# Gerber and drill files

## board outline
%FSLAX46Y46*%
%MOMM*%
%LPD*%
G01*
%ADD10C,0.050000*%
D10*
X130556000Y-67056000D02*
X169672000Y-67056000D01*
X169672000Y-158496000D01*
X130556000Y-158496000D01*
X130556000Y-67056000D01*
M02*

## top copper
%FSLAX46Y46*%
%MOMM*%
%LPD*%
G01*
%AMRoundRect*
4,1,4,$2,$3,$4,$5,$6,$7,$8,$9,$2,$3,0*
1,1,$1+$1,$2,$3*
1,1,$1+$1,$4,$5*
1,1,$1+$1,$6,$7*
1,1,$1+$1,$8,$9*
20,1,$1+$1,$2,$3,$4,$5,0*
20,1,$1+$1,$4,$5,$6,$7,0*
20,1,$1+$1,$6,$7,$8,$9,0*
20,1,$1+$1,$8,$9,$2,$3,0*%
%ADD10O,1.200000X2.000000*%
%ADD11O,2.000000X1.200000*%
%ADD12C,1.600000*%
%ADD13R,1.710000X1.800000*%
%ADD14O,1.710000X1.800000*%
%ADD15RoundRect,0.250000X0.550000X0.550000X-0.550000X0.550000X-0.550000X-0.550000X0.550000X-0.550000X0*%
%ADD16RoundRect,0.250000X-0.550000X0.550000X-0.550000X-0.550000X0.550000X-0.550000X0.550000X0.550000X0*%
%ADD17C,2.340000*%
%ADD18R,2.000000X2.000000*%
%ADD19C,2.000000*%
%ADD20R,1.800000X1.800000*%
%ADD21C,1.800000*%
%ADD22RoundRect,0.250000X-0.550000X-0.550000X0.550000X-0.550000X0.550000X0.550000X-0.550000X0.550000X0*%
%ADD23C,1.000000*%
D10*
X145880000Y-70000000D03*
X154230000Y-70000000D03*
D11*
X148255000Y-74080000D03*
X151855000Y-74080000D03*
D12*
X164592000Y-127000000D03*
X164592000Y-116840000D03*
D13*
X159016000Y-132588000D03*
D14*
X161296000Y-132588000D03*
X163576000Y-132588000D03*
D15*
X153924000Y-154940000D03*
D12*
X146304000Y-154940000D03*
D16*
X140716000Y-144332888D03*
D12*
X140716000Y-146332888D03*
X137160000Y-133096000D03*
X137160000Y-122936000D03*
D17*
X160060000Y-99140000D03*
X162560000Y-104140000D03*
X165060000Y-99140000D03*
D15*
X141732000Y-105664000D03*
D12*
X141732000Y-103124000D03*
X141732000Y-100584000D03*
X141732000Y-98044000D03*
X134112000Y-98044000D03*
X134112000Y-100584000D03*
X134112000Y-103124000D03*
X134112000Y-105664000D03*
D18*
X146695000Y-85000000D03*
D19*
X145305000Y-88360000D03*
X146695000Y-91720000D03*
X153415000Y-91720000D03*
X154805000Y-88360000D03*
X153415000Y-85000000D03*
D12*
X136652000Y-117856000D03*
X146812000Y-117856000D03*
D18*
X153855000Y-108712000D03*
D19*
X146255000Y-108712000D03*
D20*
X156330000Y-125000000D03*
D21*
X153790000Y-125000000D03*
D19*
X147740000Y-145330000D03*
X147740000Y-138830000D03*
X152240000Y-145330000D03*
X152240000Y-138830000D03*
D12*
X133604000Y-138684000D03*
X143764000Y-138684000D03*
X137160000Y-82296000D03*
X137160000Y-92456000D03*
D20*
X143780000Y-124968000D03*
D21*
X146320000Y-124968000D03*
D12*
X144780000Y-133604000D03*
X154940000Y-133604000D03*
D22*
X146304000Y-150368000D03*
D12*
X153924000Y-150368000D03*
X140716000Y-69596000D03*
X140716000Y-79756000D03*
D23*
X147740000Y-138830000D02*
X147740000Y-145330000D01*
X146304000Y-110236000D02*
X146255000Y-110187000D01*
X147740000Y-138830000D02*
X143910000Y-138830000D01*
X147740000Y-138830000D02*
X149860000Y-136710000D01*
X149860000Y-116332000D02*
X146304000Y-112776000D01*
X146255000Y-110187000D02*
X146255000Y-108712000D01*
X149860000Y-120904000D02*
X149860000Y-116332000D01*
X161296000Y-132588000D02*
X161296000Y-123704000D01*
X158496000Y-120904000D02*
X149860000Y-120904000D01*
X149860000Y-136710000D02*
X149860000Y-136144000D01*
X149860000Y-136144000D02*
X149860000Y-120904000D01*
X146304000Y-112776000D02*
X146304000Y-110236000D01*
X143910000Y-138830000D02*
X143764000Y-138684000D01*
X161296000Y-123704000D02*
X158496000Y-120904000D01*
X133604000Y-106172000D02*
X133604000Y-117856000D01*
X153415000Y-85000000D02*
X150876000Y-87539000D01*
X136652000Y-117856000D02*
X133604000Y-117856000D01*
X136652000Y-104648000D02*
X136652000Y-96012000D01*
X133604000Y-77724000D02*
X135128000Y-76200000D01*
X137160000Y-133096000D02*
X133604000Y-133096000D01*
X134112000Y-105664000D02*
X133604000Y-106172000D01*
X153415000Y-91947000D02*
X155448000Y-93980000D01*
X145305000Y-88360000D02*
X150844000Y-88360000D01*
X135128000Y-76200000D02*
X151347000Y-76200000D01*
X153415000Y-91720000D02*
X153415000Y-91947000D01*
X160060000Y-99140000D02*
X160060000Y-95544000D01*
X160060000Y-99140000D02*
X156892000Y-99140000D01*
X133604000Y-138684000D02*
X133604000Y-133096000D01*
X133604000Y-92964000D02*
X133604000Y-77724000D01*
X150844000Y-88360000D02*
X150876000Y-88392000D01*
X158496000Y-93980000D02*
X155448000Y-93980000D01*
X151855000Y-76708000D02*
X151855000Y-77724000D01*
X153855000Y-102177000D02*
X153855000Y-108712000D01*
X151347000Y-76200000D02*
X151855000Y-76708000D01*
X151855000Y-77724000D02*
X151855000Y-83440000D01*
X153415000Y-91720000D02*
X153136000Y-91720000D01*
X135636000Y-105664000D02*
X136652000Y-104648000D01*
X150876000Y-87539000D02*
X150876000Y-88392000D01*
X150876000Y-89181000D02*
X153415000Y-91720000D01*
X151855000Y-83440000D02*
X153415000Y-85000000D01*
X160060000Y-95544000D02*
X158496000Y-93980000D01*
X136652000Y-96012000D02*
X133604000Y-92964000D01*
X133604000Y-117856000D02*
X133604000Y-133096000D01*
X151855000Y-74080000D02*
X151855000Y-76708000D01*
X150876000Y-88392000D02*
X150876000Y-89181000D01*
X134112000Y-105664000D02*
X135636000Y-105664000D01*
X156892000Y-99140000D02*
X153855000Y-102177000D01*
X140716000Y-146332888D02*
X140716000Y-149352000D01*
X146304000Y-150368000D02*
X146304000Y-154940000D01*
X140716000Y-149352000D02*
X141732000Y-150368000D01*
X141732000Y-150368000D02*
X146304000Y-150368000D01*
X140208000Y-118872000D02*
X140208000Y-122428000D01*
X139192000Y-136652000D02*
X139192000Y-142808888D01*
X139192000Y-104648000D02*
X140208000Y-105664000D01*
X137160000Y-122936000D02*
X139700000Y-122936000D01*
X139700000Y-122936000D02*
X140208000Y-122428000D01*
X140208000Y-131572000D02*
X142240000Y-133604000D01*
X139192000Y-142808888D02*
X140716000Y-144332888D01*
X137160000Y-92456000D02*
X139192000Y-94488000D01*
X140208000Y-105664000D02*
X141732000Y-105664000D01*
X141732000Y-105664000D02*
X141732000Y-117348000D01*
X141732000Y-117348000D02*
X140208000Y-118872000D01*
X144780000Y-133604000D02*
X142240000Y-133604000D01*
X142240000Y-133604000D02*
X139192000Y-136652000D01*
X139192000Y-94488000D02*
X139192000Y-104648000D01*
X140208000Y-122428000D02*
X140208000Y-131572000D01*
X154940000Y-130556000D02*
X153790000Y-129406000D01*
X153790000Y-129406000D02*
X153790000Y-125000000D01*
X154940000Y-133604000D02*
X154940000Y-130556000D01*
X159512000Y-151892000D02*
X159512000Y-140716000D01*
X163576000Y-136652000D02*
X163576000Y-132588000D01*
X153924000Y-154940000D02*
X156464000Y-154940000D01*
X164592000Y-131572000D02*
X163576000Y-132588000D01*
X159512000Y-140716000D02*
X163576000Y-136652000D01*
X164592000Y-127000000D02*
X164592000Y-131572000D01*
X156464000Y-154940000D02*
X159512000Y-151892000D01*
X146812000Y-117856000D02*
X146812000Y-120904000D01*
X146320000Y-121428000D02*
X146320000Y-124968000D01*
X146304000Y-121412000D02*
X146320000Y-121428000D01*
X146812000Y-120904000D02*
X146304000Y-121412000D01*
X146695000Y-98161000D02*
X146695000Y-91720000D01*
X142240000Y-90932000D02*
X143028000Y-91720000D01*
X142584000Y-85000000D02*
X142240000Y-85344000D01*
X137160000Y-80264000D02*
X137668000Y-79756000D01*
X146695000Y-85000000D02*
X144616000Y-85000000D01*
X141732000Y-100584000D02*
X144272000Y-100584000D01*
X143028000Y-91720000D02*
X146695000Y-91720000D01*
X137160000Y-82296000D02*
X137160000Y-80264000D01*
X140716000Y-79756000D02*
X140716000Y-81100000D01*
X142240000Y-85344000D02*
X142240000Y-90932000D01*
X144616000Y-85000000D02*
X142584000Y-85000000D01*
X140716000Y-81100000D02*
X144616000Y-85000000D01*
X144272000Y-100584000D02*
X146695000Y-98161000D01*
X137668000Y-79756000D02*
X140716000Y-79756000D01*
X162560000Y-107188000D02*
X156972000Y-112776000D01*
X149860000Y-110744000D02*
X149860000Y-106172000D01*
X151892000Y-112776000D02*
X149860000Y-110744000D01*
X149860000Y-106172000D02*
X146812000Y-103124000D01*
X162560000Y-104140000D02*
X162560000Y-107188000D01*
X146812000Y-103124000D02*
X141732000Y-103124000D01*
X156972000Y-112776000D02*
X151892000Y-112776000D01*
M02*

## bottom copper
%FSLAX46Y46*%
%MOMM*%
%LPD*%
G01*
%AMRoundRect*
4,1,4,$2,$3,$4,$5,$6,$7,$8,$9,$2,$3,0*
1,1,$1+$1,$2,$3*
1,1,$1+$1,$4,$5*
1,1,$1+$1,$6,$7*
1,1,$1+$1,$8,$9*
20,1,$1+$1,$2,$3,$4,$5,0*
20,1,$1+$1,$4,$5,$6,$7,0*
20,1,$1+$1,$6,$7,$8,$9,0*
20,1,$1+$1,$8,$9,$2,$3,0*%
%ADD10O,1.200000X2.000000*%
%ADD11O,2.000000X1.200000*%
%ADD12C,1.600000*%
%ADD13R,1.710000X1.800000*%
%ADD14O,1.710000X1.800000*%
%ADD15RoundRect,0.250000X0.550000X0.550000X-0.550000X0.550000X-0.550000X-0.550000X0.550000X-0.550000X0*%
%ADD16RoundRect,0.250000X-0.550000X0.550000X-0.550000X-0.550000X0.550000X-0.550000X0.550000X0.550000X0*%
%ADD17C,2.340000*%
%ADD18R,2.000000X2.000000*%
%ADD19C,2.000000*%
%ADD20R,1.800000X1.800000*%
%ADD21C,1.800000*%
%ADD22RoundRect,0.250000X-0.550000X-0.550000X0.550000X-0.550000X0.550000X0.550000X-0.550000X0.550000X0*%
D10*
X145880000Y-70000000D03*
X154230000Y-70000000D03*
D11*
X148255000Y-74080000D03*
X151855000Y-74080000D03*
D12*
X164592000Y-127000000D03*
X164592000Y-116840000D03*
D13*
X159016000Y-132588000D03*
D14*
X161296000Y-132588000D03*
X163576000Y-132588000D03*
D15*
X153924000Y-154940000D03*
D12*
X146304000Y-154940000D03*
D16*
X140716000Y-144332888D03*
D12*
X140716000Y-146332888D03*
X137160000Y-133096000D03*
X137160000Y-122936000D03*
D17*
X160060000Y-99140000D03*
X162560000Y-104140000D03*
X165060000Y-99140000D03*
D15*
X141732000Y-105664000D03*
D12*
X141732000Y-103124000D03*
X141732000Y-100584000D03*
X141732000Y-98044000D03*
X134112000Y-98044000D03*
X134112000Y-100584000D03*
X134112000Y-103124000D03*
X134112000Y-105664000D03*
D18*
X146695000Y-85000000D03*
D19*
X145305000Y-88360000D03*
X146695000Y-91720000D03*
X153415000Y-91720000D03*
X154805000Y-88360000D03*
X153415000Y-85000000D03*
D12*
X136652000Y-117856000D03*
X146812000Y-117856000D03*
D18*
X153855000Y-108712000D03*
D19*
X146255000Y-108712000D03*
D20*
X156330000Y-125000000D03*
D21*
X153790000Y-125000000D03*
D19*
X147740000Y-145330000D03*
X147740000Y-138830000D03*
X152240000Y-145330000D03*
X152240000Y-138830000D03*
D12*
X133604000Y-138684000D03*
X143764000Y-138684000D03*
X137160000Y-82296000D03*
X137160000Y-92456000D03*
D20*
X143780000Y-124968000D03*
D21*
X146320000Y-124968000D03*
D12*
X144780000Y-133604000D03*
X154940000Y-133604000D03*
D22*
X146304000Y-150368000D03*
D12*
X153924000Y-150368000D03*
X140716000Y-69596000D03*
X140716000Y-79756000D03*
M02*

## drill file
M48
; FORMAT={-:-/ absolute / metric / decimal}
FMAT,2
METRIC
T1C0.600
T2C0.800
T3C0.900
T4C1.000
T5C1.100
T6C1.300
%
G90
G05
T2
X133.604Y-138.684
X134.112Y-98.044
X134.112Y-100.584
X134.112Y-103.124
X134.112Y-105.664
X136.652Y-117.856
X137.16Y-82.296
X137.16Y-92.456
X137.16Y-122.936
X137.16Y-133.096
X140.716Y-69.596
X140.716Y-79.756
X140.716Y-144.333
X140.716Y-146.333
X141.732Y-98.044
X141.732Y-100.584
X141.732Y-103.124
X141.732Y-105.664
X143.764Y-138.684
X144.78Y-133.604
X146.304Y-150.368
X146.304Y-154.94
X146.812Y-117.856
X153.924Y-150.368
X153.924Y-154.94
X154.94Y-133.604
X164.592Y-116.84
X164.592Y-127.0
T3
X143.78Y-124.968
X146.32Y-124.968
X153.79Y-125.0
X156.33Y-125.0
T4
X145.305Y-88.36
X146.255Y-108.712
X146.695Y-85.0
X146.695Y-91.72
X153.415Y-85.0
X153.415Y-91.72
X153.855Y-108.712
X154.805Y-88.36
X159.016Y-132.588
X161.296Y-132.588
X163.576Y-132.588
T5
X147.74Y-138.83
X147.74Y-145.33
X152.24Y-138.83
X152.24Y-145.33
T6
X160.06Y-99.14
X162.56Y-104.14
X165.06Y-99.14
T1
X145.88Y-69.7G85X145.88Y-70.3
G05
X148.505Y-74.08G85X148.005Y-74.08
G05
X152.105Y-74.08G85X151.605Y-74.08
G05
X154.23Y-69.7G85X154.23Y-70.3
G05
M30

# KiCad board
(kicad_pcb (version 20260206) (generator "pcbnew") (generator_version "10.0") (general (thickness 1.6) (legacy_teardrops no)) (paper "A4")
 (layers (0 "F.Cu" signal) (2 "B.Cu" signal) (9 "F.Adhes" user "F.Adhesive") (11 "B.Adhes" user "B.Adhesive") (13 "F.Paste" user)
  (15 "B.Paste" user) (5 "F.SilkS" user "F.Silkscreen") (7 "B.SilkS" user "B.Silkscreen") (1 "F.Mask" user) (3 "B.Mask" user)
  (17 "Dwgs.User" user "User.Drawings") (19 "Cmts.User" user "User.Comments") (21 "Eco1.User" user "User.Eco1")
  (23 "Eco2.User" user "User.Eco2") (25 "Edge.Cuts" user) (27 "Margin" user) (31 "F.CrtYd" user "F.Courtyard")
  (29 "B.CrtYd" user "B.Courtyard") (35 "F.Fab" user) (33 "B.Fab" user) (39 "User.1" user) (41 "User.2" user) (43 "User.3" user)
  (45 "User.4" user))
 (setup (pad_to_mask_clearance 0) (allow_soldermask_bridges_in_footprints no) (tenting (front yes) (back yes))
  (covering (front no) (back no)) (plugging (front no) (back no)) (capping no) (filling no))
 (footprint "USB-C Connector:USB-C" (layer "F.Cu") (at 150.055 70)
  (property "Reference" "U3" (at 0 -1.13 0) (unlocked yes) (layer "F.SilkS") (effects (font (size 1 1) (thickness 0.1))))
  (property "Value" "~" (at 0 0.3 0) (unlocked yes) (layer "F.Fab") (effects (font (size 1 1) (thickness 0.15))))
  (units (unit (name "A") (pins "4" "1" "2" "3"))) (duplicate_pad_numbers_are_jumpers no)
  (pad "1" thru_hole oval (at -4.175 0 270) (size 2 1.2) (drill oval 1.2 0.6) (layers "*.Cu" "*.Mask") (remove_unused_layers no)
   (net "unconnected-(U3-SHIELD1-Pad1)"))
  (pad "2" thru_hole oval (at 4.175 0 270) (size 2 1.2) (drill oval 1.2 0.6) (layers "*.Cu" "*.Mask") (remove_unused_layers no)
   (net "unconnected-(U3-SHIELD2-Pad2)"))
  (pad "3" thru_hole oval (at -1.8 4.08 270) (size 1.2 2) (drill oval 0.6 1.1) (layers "*.Cu" "*.Mask") (remove_unused_layers no)
   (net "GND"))
  (pad "4" thru_hole oval (at 1.8 4.08 270) (size 1.2 2) (drill oval 0.6 1.1) (layers "*.Cu" "*.Mask") (remove_unused_layers no) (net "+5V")))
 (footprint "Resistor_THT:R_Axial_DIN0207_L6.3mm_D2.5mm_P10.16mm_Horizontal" (layer "F.Cu") (at 164.592 127 90)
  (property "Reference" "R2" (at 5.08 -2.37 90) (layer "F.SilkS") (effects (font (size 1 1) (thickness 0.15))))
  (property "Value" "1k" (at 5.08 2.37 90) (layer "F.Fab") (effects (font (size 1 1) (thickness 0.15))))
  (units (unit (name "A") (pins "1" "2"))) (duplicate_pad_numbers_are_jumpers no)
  (pad "1" thru_hole circle (at 0 0 90) (size 1.6 1.6) (drill 0.8) (layers "*.Cu" "*.Mask") (remove_unused_layers no) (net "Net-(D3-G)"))
  (pad "2" thru_hole circle (at 10.16 0 90) (size 1.6 1.6) (drill 0.8) (layers "*.Cu" "*.Mask") (remove_unused_layers no) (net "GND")))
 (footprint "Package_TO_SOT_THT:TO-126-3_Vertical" (layer "F.Cu") (at 159.016 132.588)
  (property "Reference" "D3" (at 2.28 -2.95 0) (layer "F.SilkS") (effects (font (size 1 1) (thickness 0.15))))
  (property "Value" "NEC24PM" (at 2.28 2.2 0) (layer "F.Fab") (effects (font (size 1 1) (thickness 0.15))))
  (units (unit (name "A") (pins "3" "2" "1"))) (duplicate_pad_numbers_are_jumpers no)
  (pad "1" thru_hole rect (at 0 0) (size 1.71 1.8) (drill 1) (layers "*.Cu" "*.Mask") (remove_unused_layers no) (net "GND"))
  (pad "2" thru_hole oval (at 2.28 0) (size 1.71 1.8) (drill 1) (layers "*.Cu" "*.Mask") (remove_unused_layers no) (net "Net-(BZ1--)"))
  (pad "3" thru_hole oval (at 4.56 0) (size 1.71 1.8) (drill 1) (layers "*.Cu" "*.Mask") (remove_unused_layers no) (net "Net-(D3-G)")))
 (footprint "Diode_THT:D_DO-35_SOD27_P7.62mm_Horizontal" (layer "F.Cu") (at 153.924 154.94 180)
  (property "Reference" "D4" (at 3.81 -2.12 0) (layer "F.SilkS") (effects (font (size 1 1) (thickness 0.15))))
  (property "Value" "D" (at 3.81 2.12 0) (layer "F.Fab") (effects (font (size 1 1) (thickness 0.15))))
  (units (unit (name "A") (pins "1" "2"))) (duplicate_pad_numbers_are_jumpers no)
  (pad "1" thru_hole roundrect (at 0 0 180) (size 1.6 1.6) (drill 0.8) (layers "*.Cu" "*.Mask") (remove_unused_layers no)
   (roundrect_rratio 0.15625) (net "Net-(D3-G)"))
  (pad "2" thru_hole circle (at 7.62 0 180) (size 1.6 1.6) (drill 0.8) (layers "*.Cu" "*.Mask") (remove_unused_layers no) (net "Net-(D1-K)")))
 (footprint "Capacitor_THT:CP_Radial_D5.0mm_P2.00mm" (layer "F.Cu") (at 140.716 144.332888 -90)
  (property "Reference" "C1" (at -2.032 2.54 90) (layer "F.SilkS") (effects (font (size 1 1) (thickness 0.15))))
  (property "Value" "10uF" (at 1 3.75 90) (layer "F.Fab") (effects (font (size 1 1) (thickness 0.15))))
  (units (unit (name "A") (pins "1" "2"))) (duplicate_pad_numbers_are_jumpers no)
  (pad "1" thru_hole roundrect (at 0 0 270) (size 1.6 1.6) (drill 0.8) (layers "*.Cu" "*.Mask") (remove_unused_layers no)
   (roundrect_rratio 0.15625) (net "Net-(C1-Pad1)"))
  (pad "2" thru_hole circle (at 2 0 270) (size 1.6 1.6) (drill 0.8) (layers "*.Cu" "*.Mask") (remove_unused_layers no) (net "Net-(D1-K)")))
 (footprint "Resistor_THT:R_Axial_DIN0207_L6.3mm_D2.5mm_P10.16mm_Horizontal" (layer "F.Cu") (at 137.16 133.096 90)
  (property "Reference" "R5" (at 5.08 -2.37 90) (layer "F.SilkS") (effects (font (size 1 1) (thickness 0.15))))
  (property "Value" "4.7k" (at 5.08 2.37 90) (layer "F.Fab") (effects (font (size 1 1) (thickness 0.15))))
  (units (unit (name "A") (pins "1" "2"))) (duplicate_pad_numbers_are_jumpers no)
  (pad "1" thru_hole circle (at 0 0 90) (size 1.6 1.6) (drill 0.8) (layers "*.Cu" "*.Mask") (remove_unused_layers no) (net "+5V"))
  (pad "2" thru_hole circle (at 10.16 0 90) (size 1.6 1.6) (drill 0.8) (layers "*.Cu" "*.Mask") (remove_unused_layers no)
   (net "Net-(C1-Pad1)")))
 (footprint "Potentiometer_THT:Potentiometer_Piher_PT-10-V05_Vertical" (layer "F.Cu") (at 160.06 99.14 -90)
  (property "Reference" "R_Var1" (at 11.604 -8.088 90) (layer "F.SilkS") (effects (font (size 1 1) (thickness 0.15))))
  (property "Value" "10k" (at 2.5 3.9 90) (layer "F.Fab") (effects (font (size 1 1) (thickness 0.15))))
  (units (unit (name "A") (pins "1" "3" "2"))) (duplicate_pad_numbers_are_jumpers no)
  (pad "1" thru_hole circle (at 0 0 270) (size 2.34 2.34) (drill 1.3) (layers "*.Cu" "*.Mask") (remove_unused_layers no) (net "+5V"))
  (pad "2" thru_hole circle (at 5 -2.5 270) (size 2.34 2.34) (drill 1.3) (layers "*.Cu" "*.Mask") (remove_unused_layers no)
   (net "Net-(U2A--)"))
  (pad "3" thru_hole circle (at 0 -5 270) (size 2.34 2.34) (drill 1.3) (layers "*.Cu" "*.Mask") (remove_unused_layers no) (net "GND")))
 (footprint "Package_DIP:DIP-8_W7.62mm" (layer "F.Cu") (at 141.732 105.664 180)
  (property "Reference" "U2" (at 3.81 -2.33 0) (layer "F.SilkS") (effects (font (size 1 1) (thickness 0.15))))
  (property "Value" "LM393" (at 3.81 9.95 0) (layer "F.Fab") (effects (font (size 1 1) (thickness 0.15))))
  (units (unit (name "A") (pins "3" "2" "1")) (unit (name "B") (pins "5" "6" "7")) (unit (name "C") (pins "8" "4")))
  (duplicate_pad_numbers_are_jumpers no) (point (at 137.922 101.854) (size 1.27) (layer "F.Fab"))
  (pad "1" thru_hole roundrect (at 0 0 180) (size 1.6 1.6) (drill 0.8) (layers "*.Cu" "*.Mask") (remove_unused_layers no)
   (roundrect_rratio 0.15625) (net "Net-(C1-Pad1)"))
  (pad "2" thru_hole circle (at 0 2.54 180) (size 1.6 1.6) (drill 0.8) (layers "*.Cu" "*.Mask") (remove_unused_layers no)
   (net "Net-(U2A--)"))
  (pad "3" thru_hole circle (at 0 5.08 180) (size 1.6 1.6) (drill 0.8) (layers "*.Cu" "*.Mask") (remove_unused_layers no)
   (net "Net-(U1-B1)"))
  (pad "4" thru_hole circle (at 0 7.62 180) (size 1.6 1.6) (drill 0.8) (layers "*.Cu" "*.Mask") (remove_unused_layers no) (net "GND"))
  (pad "5" thru_hole circle (at 7.62 7.62 180) (size 1.6 1.6) (drill 0.8) (layers "*.Cu" "*.Mask") (remove_unused_layers no)
   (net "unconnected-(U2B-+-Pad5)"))
  (pad "6" thru_hole circle (at 7.62 5.08 180) (size 1.6 1.6) (drill 0.8) (layers "*.Cu" "*.Mask") (remove_unused_layers no)
   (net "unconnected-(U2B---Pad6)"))
  (pad "7" thru_hole circle (at 7.62 2.54 180) (size 1.6 1.6) (drill 0.8) (layers "*.Cu" "*.Mask") (remove_unused_layers no)
   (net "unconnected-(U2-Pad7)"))
  (pad "8" thru_hole circle (at 7.62 0 180) (size 1.6 1.6) (drill 0.8) (layers "*.Cu" "*.Mask") (remove_unused_layers no) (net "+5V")))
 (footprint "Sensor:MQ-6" (layer "F.Cu") (at 146.695 85)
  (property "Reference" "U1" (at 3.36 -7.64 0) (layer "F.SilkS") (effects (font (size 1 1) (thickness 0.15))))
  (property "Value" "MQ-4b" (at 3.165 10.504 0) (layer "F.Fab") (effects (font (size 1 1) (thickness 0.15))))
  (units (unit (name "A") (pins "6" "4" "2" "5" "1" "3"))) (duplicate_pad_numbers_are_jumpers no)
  (pad "1" thru_hole rect (at 0 0) (size 2 2) (drill 1) (layers "*.Cu" "*.Mask") (remove_unused_layers no) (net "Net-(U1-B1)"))
  (pad "2" thru_hole circle (at -1.39 3.36) (size 2 2) (drill 1) (layers "*.Cu" "*.Mask") (remove_unused_layers no) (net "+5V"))
  (pad "3" thru_hole circle (at 0 6.72 90) (size 2 2) (drill 1) (layers "*.Cu" "*.Mask") (remove_unused_layers no) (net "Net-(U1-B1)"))
  (pad "4" thru_hole circle (at 6.72 6.72 180) (size 2 2) (drill 1) (layers "*.Cu" "*.Mask") (remove_unused_layers no) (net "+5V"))
  (pad "5" thru_hole circle (at 8.11 3.36) (size 2 2) (drill 1) (layers "*.Cu" "*.Mask") (remove_unused_layers no) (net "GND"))
  (pad "6" thru_hole circle (at 6.72 0 270) (size 2 2) (drill 1) (layers "*.Cu" "*.Mask") (remove_unused_layers no) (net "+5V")))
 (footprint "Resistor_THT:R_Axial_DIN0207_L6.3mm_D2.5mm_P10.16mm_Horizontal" (layer "F.Cu") (at 136.652 117.856)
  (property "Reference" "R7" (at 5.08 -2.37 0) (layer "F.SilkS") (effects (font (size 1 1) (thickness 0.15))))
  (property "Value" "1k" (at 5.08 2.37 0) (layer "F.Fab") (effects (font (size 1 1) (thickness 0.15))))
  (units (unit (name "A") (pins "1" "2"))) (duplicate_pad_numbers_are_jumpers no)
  (pad "1" thru_hole circle (at 0 0) (size 1.6 1.6) (drill 0.8) (layers "*.Cu" "*.Mask") (remove_unused_layers no) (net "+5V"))
  (pad "2" thru_hole circle (at 10.16 0) (size 1.6 1.6) (drill 0.8) (layers "*.Cu" "*.Mask") (remove_unused_layers no) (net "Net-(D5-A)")))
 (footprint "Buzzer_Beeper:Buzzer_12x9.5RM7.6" (layer "F.Cu") (at 153.855 108.712 180)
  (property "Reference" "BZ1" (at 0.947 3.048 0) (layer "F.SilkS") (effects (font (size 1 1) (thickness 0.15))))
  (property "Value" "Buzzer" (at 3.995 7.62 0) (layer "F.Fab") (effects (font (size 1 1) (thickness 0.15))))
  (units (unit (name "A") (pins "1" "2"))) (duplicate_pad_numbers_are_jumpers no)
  (pad "1" thru_hole rect (at 0 0 180) (size 2 2) (drill 1) (layers "*.Cu" "*.Mask") (remove_unused_layers no) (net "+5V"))
  (pad "2" thru_hole circle (at 7.6 0 180) (size 2 2) (drill 1) (layers "*.Cu" "*.Mask") (remove_unused_layers no) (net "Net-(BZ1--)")))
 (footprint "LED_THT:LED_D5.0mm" (layer "F.Cu") (at 156.33 125 180)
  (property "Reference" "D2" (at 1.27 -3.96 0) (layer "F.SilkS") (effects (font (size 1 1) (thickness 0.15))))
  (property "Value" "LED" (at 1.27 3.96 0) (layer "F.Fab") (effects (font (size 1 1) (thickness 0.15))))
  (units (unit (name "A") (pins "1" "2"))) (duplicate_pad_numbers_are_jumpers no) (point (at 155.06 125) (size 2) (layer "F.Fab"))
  (pad "1" thru_hole rect (at 0 0 180) (size 1.8 1.8) (drill 0.9) (layers "*.Cu" "*.Mask") (remove_unused_layers no) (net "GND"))
  (pad "2" thru_hole circle (at 2.54 0 180) (size 1.8 1.8) (drill 0.9) (layers "*.Cu" "*.Mask") (remove_unused_layers no) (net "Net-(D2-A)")))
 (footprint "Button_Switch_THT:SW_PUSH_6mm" (layer "F.Cu") (at 147.74 145.33 90)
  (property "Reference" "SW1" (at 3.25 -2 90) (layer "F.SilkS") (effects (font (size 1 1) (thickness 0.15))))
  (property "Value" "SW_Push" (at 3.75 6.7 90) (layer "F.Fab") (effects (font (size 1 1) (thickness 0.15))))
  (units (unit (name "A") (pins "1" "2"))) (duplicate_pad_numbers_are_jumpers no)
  (pad "1" thru_hole circle (at 0 0 180) (size 2 2) (drill 1.1) (layers "*.Cu" "*.Mask") (remove_unused_layers no) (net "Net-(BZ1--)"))
  (pad "1" thru_hole circle (at 6.5 0 180) (size 2 2) (drill 1.1) (layers "*.Cu" "*.Mask") (remove_unused_layers no) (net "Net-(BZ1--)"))
  (pad "2" thru_hole circle (at 0 4.5 180) (size 2 2) (drill 1.1) (layers "*.Cu" "*.Mask") (remove_unused_layers no) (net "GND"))
  (pad "2" thru_hole circle (at 6.5 4.5 180) (size 2 2) (drill 1.1) (layers "*.Cu" "*.Mask") (remove_unused_layers no) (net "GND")))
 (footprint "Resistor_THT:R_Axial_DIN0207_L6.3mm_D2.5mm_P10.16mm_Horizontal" (layer "F.Cu") (at 133.604 138.684)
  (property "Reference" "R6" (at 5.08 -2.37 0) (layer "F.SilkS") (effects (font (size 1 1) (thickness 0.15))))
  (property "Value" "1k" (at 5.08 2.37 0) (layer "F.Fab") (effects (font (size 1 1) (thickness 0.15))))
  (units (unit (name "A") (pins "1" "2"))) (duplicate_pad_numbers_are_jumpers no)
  (pad "1" thru_hole circle (at 0 0) (size 1.6 1.6) (drill 0.8) (layers "*.Cu" "*.Mask") (remove_unused_layers no) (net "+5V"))
  (pad "2" thru_hole circle (at 10.16 0) (size 1.6 1.6) (drill 0.8) (layers "*.Cu" "*.Mask") (remove_unused_layers no) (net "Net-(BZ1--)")))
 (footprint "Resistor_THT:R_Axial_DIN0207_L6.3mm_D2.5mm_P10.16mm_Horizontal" (layer "F.Cu") (at 137.16 82.296 -90)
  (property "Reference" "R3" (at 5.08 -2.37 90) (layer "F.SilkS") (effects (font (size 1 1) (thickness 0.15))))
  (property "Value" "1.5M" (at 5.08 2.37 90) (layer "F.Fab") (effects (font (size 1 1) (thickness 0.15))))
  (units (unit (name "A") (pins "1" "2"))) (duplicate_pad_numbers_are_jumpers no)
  (pad "1" thru_hole circle (at 0 0 270) (size 1.6 1.6) (drill 0.8) (layers "*.Cu" "*.Mask") (remove_unused_layers no) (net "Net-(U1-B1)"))
  (pad "2" thru_hole circle (at 10.16 0 270) (size 1.6 1.6) (drill 0.8) (layers "*.Cu" "*.Mask") (remove_unused_layers no)
   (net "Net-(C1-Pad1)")))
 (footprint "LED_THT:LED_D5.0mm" (layer "F.Cu") (at 143.78 124.968)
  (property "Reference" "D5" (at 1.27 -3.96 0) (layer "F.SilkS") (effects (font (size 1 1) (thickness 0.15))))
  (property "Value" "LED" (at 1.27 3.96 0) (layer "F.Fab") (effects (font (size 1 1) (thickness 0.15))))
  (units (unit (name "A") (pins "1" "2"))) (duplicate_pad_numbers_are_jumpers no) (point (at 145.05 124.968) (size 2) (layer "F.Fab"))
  (pad "1" thru_hole rect (at 0 0) (size 1.8 1.8) (drill 0.9) (layers "*.Cu" "*.Mask") (remove_unused_layers no) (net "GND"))
  (pad "2" thru_hole circle (at 2.54 0) (size 1.8 1.8) (drill 0.9) (layers "*.Cu" "*.Mask") (remove_unused_layers no) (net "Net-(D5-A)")))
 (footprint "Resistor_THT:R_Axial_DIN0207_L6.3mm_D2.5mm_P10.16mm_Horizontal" (layer "F.Cu") (at 144.78 133.604)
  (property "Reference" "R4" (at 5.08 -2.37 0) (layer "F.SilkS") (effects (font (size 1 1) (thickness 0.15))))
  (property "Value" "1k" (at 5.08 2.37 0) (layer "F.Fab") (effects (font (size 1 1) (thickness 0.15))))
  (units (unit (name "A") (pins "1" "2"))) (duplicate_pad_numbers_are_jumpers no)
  (pad "1" thru_hole circle (at 0 0) (size 1.6 1.6) (drill 0.8) (layers "*.Cu" "*.Mask") (remove_unused_layers no) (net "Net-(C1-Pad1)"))
  (pad "2" thru_hole circle (at 10.16 0) (size 1.6 1.6) (drill 0.8) (layers "*.Cu" "*.Mask") (remove_unused_layers no) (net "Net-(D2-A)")))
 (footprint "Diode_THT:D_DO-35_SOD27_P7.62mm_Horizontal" (layer "F.Cu") (at 146.304 150.368)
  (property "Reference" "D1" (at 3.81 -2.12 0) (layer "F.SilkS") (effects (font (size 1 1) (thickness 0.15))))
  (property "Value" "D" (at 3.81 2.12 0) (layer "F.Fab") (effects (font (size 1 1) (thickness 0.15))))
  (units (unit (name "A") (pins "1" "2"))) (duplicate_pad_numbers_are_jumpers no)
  (pad "1" thru_hole roundrect (at 0 0) (size 1.6 1.6) (drill 0.8) (layers "*.Cu" "*.Mask") (remove_unused_layers no)
   (roundrect_rratio 0.15625) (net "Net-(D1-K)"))
  (pad "2" thru_hole circle (at 7.62 0) (size 1.6 1.6) (drill 0.8) (layers "*.Cu" "*.Mask") (remove_unused_layers no) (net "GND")))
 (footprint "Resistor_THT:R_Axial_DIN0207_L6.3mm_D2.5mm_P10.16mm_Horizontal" (layer "F.Cu") (at 140.716 69.596 -90)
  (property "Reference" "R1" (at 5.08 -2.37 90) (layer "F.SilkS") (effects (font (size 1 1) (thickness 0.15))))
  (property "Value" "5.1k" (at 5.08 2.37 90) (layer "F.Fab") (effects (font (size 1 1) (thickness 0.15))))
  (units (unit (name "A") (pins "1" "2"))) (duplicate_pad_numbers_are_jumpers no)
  (pad "1" thru_hole circle (at 0 0 270) (size 1.6 1.6) (drill 0.8) (layers "*.Cu" "*.Mask") (remove_unused_layers no) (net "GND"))
  (pad "2" thru_hole circle (at 10.16 0 270) (size 1.6 1.6) (drill 0.8) (layers "*.Cu" "*.Mask") (remove_unused_layers no)
   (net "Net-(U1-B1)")))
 (gr_rect (start 130.556 67.056) (end 169.672 158.496) (stroke (width 0.05) (type default)) (fill no) (layer "Edge.Cuts"))
 (segment (start 147.74 138.83) (end 147.74 145.33) (width 1) (layer "F.Cu") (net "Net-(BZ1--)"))
 (segment (start 146.304 110.236) (end 146.255 110.187) (width 1) (layer "F.Cu") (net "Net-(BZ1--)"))
 (segment (start 147.74 138.83) (end 143.91 138.83) (width 1) (layer "F.Cu") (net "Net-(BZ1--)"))
 (segment (start 147.74 138.83) (end 149.86 136.71) (width 1) (layer "F.Cu") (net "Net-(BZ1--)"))
 (segment (start 149.86 116.332) (end 146.304 112.776) (width 1) (layer "F.Cu") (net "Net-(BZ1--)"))
 (segment (start 146.255 110.187) (end 146.255 108.712) (width 1) (layer "F.Cu") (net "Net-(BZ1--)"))
 (segment (start 149.86 120.904) (end 149.86 116.332) (width 1) (layer "F.Cu") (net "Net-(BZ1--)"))
 (segment (start 161.296 132.588) (end 161.296 123.704) (width 1) (layer "F.Cu") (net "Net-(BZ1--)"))
 (segment (start 158.496 120.904) (end 149.86 120.904) (width 1) (layer "F.Cu") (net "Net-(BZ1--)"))
 (segment (start 149.86 136.71) (end 149.86 136.144) (width 1) (layer "F.Cu") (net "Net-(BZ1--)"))
 (segment (start 149.86 136.144) (end 149.86 120.904) (width 1) (layer "F.Cu") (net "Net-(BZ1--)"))
 (segment (start 146.304 112.776) (end 146.304 110.236) (width 1) (layer "F.Cu") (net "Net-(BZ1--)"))
 (segment (start 143.91 138.83) (end 143.764 138.684) (width 1) (layer "F.Cu") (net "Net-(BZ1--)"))
 (segment (start 161.296 123.704) (end 158.496 120.904) (width 1) (layer "F.Cu") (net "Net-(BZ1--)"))
 (segment (start 133.604 106.172) (end 133.604 117.856) (width 1) (layer "F.Cu") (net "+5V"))
 (segment (start 153.415 85) (end 150.876 87.539) (width 1) (layer "F.Cu") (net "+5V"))
 (segment (start 136.652 117.856) (end 133.604 117.856) (width 1) (layer "F.Cu") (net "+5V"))
 (segment (start 136.652 104.648) (end 136.652 96.012) (width 1) (layer "F.Cu") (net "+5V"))
 (segment (start 133.604 77.724) (end 135.128 76.2) (width 1) (layer "F.Cu") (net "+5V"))
 (segment (start 137.16 133.096) (end 133.604 133.096) (width 1) (layer "F.Cu") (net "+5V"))
 (segment (start 134.112 105.664) (end 133.604 106.172) (width 1) (layer "F.Cu") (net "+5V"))
 (segment (start 153.415 91.947) (end 155.448 93.98) (width 1) (layer "F.Cu") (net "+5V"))
 (segment (start 145.305 88.36) (end 150.844 88.36) (width 1) (layer "F.Cu") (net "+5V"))
 (segment (start 135.128 76.2) (end 151.347 76.2) (width 1) (layer "F.Cu") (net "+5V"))
 (segment (start 153.415 91.72) (end 153.415 91.947) (width 1) (layer "F.Cu") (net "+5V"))
 (segment (start 160.06 99.14) (end 160.06 95.544) (width 1) (layer "F.Cu") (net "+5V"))
 (segment (start 160.06 99.14) (end 156.892 99.14) (width 1) (layer "F.Cu") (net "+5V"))
 (segment (start 133.604 138.684) (end 133.604 133.096) (width 1) (layer "F.Cu") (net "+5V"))
 (segment (start 133.604 92.964) (end 133.604 77.724) (width 1) (layer "F.Cu") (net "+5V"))
 (segment (start 150.844 88.36) (end 150.876 88.392) (width 1) (layer "F.Cu") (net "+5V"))
 (segment (start 158.496 93.98) (end 155.448 93.98) (width 1) (layer "F.Cu") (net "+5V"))
 (segment (start 151.855 76.708) (end 151.855 77.724) (width 1) (layer "F.Cu") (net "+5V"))
 (segment (start 153.855 102.177) (end 153.855 108.712) (width 1) (layer "F.Cu") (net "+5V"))
 (segment (start 151.347 76.2) (end 151.855 76.708) (width 1) (layer "F.Cu") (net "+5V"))
 (segment (start 151.855 77.724) (end 151.855 83.44) (width 1) (layer "F.Cu") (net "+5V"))
 (segment (start 153.415 91.72) (end 153.136 91.72) (width 1) (layer "F.Cu") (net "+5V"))
 (segment (start 135.636 105.664) (end 136.652 104.648) (width 1) (layer "F.Cu") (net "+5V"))
 (segment (start 150.876 87.539) (end 150.876 88.392) (width 1) (layer "F.Cu") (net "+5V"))
 (segment (start 150.876 89.181) (end 153.415 91.72) (width 1) (layer "F.Cu") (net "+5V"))
 (segment (start 151.855 83.44) (end 153.415 85) (width 1) (layer "F.Cu") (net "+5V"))
 (segment (start 160.06 95.544) (end 158.496 93.98) (width 1) (layer "F.Cu") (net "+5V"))
 (segment (start 136.652 96.012) (end 133.604 92.964) (width 1) (layer "F.Cu") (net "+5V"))
 (segment (start 133.604 117.856) (end 133.604 133.096) (width 1) (layer "F.Cu") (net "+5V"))
 (segment (start 151.855 74.08) (end 151.855 76.708) (width 1) (layer "F.Cu") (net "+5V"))
 (segment (start 150.876 88.392) (end 150.876 89.181) (width 1) (layer "F.Cu") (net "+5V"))
 (segment (start 134.112 105.664) (end 135.636 105.664) (width 1) (layer "F.Cu") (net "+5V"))
 (segment (start 156.892 99.14) (end 153.855 102.177) (width 1) (layer "F.Cu") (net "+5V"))
 (segment (start 140.716 146.332888) (end 140.716 149.352) (width 1) (layer "F.Cu") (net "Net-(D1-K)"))
 (segment (start 146.304 150.368) (end 146.304 154.94) (width 1) (layer "F.Cu") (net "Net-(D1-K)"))
 (segment (start 140.716 149.352) (end 141.732 150.368) (width 1) (layer "F.Cu") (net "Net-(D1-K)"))
 (segment (start 141.732 150.368) (end 146.304 150.368) (width 1) (layer "F.Cu") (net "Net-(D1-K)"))
 (segment (start 140.208 118.872) (end 140.208 122.428) (width 1) (layer "F.Cu") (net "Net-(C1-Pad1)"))
 (segment (start 139.192 136.652) (end 139.192 142.808888) (width 1) (layer "F.Cu") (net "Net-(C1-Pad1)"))
 (segment (start 139.192 104.648) (end 140.208 105.664) (width 1) (layer "F.Cu") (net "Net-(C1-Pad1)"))
 (segment (start 137.16 122.936) (end 139.7 122.936) (width 1) (layer "F.Cu") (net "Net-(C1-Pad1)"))
 (segment (start 139.7 122.936) (end 140.208 122.428) (width 1) (layer "F.Cu") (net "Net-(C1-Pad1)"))
 (segment (start 140.208 131.572) (end 142.24 133.604) (width 1) (layer "F.Cu") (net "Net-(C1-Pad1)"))
 (segment (start 139.192 142.808888) (end 140.716 144.332888) (width 1) (layer "F.Cu") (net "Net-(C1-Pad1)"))
 (segment (start 137.16 92.456) (end 139.192 94.488) (width 1) (layer "F.Cu") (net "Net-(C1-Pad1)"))
 (segment (start 140.208 105.664) (end 141.732 105.664) (width 1) (layer "F.Cu") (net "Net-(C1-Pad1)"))
 (segment (start 141.732 105.664) (end 141.732 117.348) (width 1) (layer "F.Cu") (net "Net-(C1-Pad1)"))
 (segment (start 141.732 117.348) (end 140.208 118.872) (width 1) (layer "F.Cu") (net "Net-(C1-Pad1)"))
 (segment (start 144.78 133.604) (end 142.24 133.604) (width 1) (layer "F.Cu") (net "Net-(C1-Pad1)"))
 (segment (start 142.24 133.604) (end 139.192 136.652) (width 1) (layer "F.Cu") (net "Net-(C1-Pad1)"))
 (segment (start 139.192 94.488) (end 139.192 104.648) (width 1) (layer "F.Cu") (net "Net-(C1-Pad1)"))
 (segment (start 140.208 122.428) (end 140.208 131.572) (width 1) (layer "F.Cu") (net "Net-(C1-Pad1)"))
 (segment (start 154.94 130.556) (end 153.79 129.406) (width 1) (layer "F.Cu") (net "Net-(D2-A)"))
 (segment (start 153.79 129.406) (end 153.79 125) (width 1) (layer "F.Cu") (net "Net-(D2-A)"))
 (segment (start 154.94 133.604) (end 154.94 130.556) (width 1) (layer "F.Cu") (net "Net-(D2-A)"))
 (segment (start 159.512 151.892) (end 159.512 140.716) (width 1) (layer "F.Cu") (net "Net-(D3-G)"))
 (segment (start 163.576 136.652) (end 163.576 132.588) (width 1) (layer "F.Cu") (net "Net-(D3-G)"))
 (segment (start 153.924 154.94) (end 156.464 154.94) (width 1) (layer "F.Cu") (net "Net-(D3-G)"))
 (segment (start 164.592 131.572) (end 163.576 132.588) (width 1) (layer "F.Cu") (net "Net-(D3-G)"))
 (segment (start 159.512 140.716) (end 163.576 136.652) (width 1) (layer "F.Cu") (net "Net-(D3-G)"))
 (segment (start 164.592 127) (end 164.592 131.572) (width 1) (layer "F.Cu") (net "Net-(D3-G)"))
 (segment (start 156.464 154.94) (end 159.512 151.892) (width 1) (layer "F.Cu") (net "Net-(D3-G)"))
 (segment (start 146.812 117.856) (end 146.812 120.904) (width 1) (layer "F.Cu") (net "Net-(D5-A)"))
 (segment (start 146.32 121.428) (end 146.32 124.968) (width 1) (layer "F.Cu") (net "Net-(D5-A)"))
 (segment (start 146.304 121.412) (end 146.32 121.428) (width 1) (layer "F.Cu") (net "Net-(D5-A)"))
 (segment (start 146.812 120.904) (end 146.304 121.412) (width 1) (layer "F.Cu") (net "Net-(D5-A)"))
 (segment (start 146.695 98.161) (end 146.695 91.72) (width 1) (layer "F.Cu") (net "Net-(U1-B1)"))
 (segment (start 142.24 90.932) (end 143.028 91.72) (width 1) (layer "F.Cu") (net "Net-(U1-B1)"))
 (segment (start 142.584 85) (end 142.24 85.344) (width 1) (layer "F.Cu") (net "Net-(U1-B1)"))
 (segment (start 137.16 80.264) (end 137.668 79.756) (width 1) (layer "F.Cu") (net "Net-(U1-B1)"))
 (segment (start 146.695 85) (end 144.616 85) (width 1) (layer "F.Cu") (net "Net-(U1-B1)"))
 (segment (start 141.732 100.584) (end 144.272 100.584) (width 1) (layer "F.Cu") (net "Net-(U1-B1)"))
 (segment (start 143.028 91.72) (end 146.695 91.72) (width 1) (layer "F.Cu") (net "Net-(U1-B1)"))
 (segment (start 137.16 82.296) (end 137.16 80.264) (width 1) (layer "F.Cu") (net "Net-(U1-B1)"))
 (segment (start 140.716 79.756) (end 140.716 81.1) (width 1) (layer "F.Cu") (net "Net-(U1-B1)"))
 (segment (start 142.24 85.344) (end 142.24 90.932) (width 1) (layer "F.Cu") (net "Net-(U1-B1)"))
 (segment (start 144.616 85) (end 142.584 85) (width 1) (layer "F.Cu") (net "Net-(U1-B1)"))
 (segment (start 140.716 81.1) (end 144.616 85) (width 1) (layer "F.Cu") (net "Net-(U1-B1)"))
 (segment (start 144.272 100.584) (end 146.695 98.161) (width 1) (layer "F.Cu") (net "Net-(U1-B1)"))
 (segment (start 137.668 79.756) (end 140.716 79.756) (width 1) (layer "F.Cu") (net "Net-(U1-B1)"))
 (segment (start 162.56 107.188) (end 156.972 112.776) (width 1) (layer "F.Cu") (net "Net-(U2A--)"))
 (segment (start 149.86 110.744) (end 149.86 106.172) (width 1) (layer "F.Cu") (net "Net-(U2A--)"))
 (segment (start 151.892 112.776) (end 149.86 110.744) (width 1) (layer "F.Cu") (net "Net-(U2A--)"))
 (segment (start 149.86 106.172) (end 146.812 103.124) (width 1) (layer "F.Cu") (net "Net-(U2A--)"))
 (segment (start 162.56 104.14) (end 162.56 107.188) (width 1) (layer "F.Cu") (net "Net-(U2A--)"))
 (segment (start 146.812 103.124) (end 141.732 103.124) (width 1) (layer "F.Cu") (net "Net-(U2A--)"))
 (segment (start 156.972 112.776) (end 151.892 112.776) (width 1) (layer "F.Cu") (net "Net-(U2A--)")))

